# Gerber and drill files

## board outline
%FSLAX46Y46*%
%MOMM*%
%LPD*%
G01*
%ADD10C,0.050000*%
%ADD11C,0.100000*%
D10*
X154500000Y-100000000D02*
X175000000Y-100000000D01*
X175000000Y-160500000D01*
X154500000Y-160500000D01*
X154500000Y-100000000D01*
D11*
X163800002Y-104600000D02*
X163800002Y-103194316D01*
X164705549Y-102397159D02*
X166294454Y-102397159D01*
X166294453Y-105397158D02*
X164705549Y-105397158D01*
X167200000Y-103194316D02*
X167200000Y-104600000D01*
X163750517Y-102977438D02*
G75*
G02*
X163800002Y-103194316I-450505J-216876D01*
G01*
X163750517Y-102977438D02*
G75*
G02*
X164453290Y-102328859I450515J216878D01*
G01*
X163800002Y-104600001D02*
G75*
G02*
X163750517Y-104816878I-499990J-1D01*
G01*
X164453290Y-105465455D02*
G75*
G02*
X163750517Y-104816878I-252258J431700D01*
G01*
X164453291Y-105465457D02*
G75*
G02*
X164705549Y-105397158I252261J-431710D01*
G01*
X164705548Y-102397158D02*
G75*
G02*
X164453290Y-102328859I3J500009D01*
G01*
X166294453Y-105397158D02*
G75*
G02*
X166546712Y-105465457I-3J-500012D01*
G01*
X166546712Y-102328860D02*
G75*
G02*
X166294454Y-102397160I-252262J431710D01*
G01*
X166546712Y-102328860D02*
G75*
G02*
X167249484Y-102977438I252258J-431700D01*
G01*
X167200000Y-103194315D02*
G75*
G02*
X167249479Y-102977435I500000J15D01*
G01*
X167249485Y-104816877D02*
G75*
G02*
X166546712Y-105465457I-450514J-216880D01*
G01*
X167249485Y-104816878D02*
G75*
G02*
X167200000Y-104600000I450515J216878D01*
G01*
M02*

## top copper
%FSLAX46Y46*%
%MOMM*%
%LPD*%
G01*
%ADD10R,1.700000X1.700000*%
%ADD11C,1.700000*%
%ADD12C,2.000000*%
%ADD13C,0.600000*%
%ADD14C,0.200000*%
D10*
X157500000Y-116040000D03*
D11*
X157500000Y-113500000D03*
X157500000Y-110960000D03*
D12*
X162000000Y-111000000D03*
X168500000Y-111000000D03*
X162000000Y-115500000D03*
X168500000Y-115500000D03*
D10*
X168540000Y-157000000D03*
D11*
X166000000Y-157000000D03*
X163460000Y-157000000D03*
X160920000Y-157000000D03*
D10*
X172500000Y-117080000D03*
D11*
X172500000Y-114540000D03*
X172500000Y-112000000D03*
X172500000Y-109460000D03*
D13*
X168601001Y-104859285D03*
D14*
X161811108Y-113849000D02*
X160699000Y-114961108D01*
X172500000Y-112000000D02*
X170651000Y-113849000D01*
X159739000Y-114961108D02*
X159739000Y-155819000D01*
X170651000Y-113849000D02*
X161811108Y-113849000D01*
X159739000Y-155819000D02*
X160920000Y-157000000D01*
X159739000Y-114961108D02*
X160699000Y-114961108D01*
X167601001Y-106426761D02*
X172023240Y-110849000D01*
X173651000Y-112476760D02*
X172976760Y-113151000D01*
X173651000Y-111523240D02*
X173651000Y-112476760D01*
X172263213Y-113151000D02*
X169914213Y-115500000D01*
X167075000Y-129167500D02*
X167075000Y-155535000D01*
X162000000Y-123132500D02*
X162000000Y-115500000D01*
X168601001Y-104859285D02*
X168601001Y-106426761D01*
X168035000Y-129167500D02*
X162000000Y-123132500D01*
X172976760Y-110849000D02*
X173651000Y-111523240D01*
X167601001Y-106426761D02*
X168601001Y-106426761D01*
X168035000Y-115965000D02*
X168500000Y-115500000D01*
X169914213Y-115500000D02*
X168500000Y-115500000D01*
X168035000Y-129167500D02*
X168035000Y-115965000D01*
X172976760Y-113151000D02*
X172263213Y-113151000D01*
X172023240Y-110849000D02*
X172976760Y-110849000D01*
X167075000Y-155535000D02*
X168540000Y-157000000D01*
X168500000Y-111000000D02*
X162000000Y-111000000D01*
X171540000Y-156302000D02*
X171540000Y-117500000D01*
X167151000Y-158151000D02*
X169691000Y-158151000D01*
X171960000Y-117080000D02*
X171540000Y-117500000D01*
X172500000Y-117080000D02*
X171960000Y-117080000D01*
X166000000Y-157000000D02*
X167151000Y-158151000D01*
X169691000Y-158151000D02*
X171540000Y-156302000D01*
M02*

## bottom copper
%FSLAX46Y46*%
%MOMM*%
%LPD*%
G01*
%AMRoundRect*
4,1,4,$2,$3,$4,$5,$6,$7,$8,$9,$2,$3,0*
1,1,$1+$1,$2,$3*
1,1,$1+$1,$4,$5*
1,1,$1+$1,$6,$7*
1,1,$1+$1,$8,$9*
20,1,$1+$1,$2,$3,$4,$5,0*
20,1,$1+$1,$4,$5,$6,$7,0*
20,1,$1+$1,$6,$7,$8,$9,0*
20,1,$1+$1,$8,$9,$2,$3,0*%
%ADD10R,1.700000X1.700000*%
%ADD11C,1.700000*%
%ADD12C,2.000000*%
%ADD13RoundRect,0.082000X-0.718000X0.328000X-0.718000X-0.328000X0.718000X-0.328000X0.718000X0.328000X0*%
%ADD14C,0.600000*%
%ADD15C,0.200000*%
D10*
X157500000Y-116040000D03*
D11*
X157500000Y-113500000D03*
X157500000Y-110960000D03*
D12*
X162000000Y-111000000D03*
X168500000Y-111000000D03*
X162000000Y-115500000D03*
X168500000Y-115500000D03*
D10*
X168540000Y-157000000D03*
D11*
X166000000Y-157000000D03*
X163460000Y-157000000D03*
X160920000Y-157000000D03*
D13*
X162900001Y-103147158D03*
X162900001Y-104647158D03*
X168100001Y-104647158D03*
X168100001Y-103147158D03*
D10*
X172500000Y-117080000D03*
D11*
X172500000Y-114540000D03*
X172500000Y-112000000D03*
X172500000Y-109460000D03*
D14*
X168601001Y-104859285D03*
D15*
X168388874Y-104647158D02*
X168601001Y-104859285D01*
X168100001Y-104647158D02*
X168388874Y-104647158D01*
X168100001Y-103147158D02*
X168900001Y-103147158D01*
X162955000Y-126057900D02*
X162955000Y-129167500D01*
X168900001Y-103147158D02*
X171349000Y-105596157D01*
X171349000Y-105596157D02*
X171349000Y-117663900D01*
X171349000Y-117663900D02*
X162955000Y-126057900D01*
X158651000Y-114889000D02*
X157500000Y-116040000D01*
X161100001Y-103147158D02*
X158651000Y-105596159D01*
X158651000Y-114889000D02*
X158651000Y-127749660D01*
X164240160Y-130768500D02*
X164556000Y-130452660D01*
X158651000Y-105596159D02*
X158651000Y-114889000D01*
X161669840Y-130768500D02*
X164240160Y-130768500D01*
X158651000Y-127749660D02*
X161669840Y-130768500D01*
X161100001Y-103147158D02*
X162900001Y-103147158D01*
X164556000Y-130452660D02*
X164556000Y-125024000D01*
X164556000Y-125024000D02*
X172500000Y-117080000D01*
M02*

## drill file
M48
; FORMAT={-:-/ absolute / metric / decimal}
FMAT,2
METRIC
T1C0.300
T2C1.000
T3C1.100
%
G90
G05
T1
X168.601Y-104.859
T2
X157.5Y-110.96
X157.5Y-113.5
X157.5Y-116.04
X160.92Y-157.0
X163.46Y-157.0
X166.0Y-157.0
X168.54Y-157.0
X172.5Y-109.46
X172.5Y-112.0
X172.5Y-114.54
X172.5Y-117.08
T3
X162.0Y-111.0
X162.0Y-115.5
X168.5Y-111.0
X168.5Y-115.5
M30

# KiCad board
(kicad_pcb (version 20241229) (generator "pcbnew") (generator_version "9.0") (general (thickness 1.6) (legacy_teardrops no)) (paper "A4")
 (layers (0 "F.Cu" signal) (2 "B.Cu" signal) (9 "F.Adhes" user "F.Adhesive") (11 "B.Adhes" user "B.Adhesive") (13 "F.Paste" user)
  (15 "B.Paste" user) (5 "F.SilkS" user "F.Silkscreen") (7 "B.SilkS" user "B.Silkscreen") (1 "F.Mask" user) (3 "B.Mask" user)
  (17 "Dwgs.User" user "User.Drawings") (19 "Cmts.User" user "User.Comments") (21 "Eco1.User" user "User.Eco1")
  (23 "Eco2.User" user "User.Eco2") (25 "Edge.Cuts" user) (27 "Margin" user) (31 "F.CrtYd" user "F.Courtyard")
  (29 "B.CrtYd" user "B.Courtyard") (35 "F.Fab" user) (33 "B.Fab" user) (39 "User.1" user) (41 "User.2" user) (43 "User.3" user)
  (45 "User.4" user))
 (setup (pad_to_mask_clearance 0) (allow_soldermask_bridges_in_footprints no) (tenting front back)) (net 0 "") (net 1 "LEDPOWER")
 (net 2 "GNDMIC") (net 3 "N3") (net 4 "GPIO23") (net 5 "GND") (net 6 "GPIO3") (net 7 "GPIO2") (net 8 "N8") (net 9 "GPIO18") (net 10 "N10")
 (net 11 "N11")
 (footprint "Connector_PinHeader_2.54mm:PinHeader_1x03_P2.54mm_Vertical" (layer "F.Cu") (at 157.5 116.04 180)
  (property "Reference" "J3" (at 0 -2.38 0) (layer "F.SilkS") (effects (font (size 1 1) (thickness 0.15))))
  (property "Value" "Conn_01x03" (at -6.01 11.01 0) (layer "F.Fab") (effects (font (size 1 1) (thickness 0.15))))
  (pad "1" thru_hole rect (at 0 0 180) (size 1.7 1.7) (drill 1) (layers "*.Cu" "*.Mask") (remove_unused_layers no) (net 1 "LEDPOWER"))
  (pad "2" thru_hole circle (at 0 2.54 180) (size 1.7 1.7) (drill 1) (layers "*.Cu" "*.Mask") (remove_unused_layers no) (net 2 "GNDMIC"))
  (pad "3" thru_hole circle (at 0 5.08 180) (size 1.7 1.7) (drill 1) (layers "*.Cu" "*.Mask") (remove_unused_layers no) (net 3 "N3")))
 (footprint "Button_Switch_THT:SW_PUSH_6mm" (layer "F.Cu") (at 162 111)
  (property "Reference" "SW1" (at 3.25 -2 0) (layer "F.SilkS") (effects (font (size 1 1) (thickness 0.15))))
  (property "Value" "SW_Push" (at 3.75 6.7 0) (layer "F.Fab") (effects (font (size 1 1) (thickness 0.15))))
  (pad "1" thru_hole circle (at 0 0 90) (size 2 2) (drill 1.1) (layers "*.Cu" "*.Mask") (remove_unused_layers no) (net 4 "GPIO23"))
  (pad "1" thru_hole circle (at 6.5 0 90) (size 2 2) (drill 1.1) (layers "*.Cu" "*.Mask") (remove_unused_layers no) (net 4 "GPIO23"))
  (pad "2" thru_hole circle (at 0 4.5 90) (size 2 2) (drill 1.1) (layers "*.Cu" "*.Mask") (remove_unused_layers no) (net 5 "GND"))
  (pad "2" thru_hole circle (at 6.5 4.5 90) (size 2 2) (drill 1.1) (layers "*.Cu" "*.Mask") (remove_unused_layers no) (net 5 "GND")))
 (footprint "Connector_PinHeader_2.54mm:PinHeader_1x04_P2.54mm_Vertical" (layer "F.Cu") (at 168.54 157 -90)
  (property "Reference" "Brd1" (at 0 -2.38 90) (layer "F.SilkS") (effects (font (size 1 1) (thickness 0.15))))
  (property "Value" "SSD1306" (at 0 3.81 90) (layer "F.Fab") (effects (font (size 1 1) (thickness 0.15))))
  (pad "1" thru_hole rect (at 0 0 270) (size 1.7 1.7) (drill 1) (layers "*.Cu" "*.Mask") (remove_unused_layers no) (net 5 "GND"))
  (pad "2" thru_hole circle (at 0 2.54 270) (size 1.7 1.7) (drill 1) (layers "*.Cu" "*.Mask") (remove_unused_layers no) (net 1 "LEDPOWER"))
  (pad "3" thru_hole circle (at 0 5.08 270) (size 1.7 1.7) (drill 1) (layers "*.Cu" "*.Mask") (remove_unused_layers no) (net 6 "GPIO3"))
  (pad "4" thru_hole circle (at 0 7.62 270) (size 1.7 1.7) (drill 1) (layers "*.Cu" "*.Mask") (remove_unused_layers no) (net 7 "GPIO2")))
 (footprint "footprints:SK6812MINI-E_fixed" (layer "F.Cu") (at 165.5 104)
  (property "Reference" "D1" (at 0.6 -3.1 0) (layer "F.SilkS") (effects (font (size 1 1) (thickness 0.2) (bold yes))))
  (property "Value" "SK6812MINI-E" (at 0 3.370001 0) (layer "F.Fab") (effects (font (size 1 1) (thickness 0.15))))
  (fp_line (start -1.699998 0.6) (end -1.699998 -0.805684) (stroke (width 0.1) (type solid)) (layer "Edge.Cuts"))
  (fp_line (start -0.794451 -1.602841) (end 0.794454 -1.602841) (stroke (width 0.1) (type solid)) (layer "Edge.Cuts"))
  (fp_line (start 0.794453 1.397158) (end -0.794451 1.397158) (stroke (width 0.1) (type solid)) (layer "Edge.Cuts"))
  (fp_line (start 1.7 -0.805684) (end 1.7 0.6) (stroke (width 0.1) (type solid)) (layer "Edge.Cuts"))
  (fp_arc (start -1.749483 -1.022562) (mid -1.712526 -0.91691) (end -1.699998 -0.805684) (stroke (width 0.1) (type solid))
   (layer "Edge.Cuts"))
  (fp_arc (start -1.749483 -1.022562) (mid -1.63807 -1.606877) (end -1.04671 -1.671141) (stroke (width 0.1) (type solid))
   (layer "Edge.Cuts"))
  (fp_arc (start -1.699998 0.600001) (mid -1.712526 0.711226) (end -1.749483 0.816878) (stroke (width 0.1) (type solid)) (layer "Edge.Cuts"))
  (fp_arc (start -1.04671 1.465455) (mid -1.638069 1.401192) (end -1.749483 0.816878) (stroke (width 0.1) (type solid)) (layer "Edge.Cuts"))
  (fp_arc (start -1.046709 1.465457) (mid -0.925121 1.414535) (end -0.794451 1.397158) (stroke (width 0.1) (type solid)) (layer "Edge.Cuts"))
  (fp_arc (start -0.794452 -1.602842) (mid -0.925122 -1.620219) (end -1.04671 -1.671141) (stroke (width 0.1) (type solid))
   (layer "Edge.Cuts"))
  (fp_arc (start 0.794453 1.397158) (mid 0.925124 1.414535) (end 1.046712 1.465457) (stroke (width 0.1) (type solid)) (layer "Edge.Cuts"))
  (fp_arc (start 1.046712 -1.67114) (mid 0.925124 -1.620218) (end 0.794454 -1.602841) (stroke (width 0.1) (type solid)) (layer "Edge.Cuts"))
  (fp_arc (start 1.046712 -1.67114) (mid 1.638072 -1.606876) (end 1.749485 -1.022562) (stroke (width 0.1) (type solid)) (layer "Edge.Cuts"))
  (fp_arc (start 1.7 -0.805685) (mid 1.712528 -0.91691) (end 1.749485 -1.022562) (stroke (width 0.1) (type solid)) (layer "Edge.Cuts"))
  (fp_arc (start 1.749485 0.816877) (mid 1.638073 1.401193) (end 1.046712 1.465457) (stroke (width 0.1) (type solid)) (layer "Edge.Cuts"))
  (fp_arc (start 1.749485 0.816878) (mid 1.712528 0.711226) (end 1.7 0.6) (stroke (width 0.1) (type solid)) (layer "Edge.Cuts"))
  (pad "1" smd roundrect (at -2.599999 -0.852842 270) (size 0.82 1.6) (layers "B.Cu" "B.Mask" "B.Paste") (roundrect_rratio 0.1)
   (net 1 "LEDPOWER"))
  (pad "2" smd roundrect (at -2.599999 0.647158 270) (size 0.82 1.6) (layers "B.Cu" "B.Mask" "B.Paste") (roundrect_rratio 0.1) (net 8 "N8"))
  (pad "3" smd roundrect (at 2.600001 0.647158 270) (size 0.82 1.6) (layers "B.Cu" "B.Mask" "B.Paste") (roundrect_rratio 0.1) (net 5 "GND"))
  (pad "4" smd roundrect (at 2.600001 -0.852842 270) (size 0.82 1.6) (layers "B.Cu" "B.Mask" "B.Paste") (roundrect_rratio 0.1)
   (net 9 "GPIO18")))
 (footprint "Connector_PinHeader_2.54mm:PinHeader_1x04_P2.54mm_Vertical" (layer "F.Cu") (at 172.5 117.08 180)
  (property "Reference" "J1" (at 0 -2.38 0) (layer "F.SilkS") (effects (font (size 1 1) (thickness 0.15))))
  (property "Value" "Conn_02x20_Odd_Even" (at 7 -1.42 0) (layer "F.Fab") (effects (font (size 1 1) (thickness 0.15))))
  (pad "1" thru_hole rect (at 0 0 180) (size 1.7 1.7) (drill 1) (layers "*.Cu" "*.Mask") (remove_unused_layers no) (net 1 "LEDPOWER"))
  (pad "2" thru_hole circle (at 0 2.54 180) (size 1.7 1.7) (drill 1) (layers "*.Cu" "*.Mask") (remove_unused_layers no) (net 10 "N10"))
  (pad "3" thru_hole circle (at 0 5.08 180) (size 1.7 1.7) (drill 1) (layers "*.Cu" "*.Mask") (remove_unused_layers no) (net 7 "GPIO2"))
  (pad "4" thru_hole circle (at 0 7.62 180) (size 1.7 1.7) (drill 1) (layers "*.Cu" "*.Mask") (remove_unused_layers no) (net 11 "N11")))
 (gr_rect (start 154.5 100) (end 175 160.5) (stroke (width 0.05) (type default)) (fill no) (layer "Edge.Cuts"))
 (segment (start 161.811108 113.849) (end 160.699 114.961108) (width 0.2) (layer "F.Cu") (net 7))
 (segment (start 172.5 112) (end 170.651 113.849) (width 0.2) (layer "F.Cu") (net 7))
 (segment (start 159.739 114.961108) (end 159.739 155.819) (width 0.2) (layer "F.Cu") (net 7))
 (segment (start 170.651 113.849) (end 161.811108 113.849) (width 0.2) (layer "F.Cu") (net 7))
 (segment (start 159.739 155.819) (end 160.92 157) (width 0.2) (layer "F.Cu") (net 7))
 (segment (start 159.739 114.961108) (end 160.699 114.961108) (width 0.2) (layer "F.Cu") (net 7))
 (segment (start 167.601001 106.426761) (end 172.02324 110.849) (width 0.2) (layer "F.Cu") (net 5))
 (segment (start 173.651 112.47676) (end 172.97676 113.151) (width 0.2) (layer "F.Cu") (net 5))
 (segment (start 173.651 111.52324) (end 173.651 112.47676) (width 0.2) (layer "F.Cu") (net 5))
 (segment (start 172.263213 113.151) (end 169.914213 115.5) (width 0.2) (layer "F.Cu") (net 5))
 (segment (start 167.075 129.1675) (end 167.075 155.535) (width 0.2) (layer "F.Cu") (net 5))
 (segment (start 162 123.1325) (end 162 115.5) (width 0.2) (layer "F.Cu") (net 5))
 (segment (start 168.601001 104.859285) (end 168.601001 106.426761) (width 0.2) (layer "F.Cu") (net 5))
 (segment (start 168.035 129.1675) (end 162 123.1325) (width 0.2) (layer "F.Cu") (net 5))
 (segment (start 172.97676 110.849) (end 173.651 111.52324) (width 0.2) (layer "F.Cu") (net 5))
 (segment (start 167.601001 106.426761) (end 168.601001 106.426761) (width 0.2) (layer "F.Cu") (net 5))
 (segment (start 168.035 115.965) (end 168.5 115.5) (width 0.2) (layer "F.Cu") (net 5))
 (segment (start 169.914213 115.5) (end 168.5 115.5) (width 0.2) (layer "F.Cu") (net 5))
 (segment (start 168.035 129.1675) (end 168.035 115.965) (width 0.2) (layer "F.Cu") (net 5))
 (segment (start 172.97676 113.151) (end 172.263213 113.151) (width 0.2) (layer "F.Cu") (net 5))
 (segment (start 172.02324 110.849) (end 172.97676 110.849) (width 0.2) (layer "F.Cu") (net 5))
 (segment (start 167.075 155.535) (end 168.54 157) (width 0.2) (layer "F.Cu") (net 5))
 (via (at 168.601001 104.859285) (size 0.6) (drill 0.3) (layers "F.Cu" "B.Cu") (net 5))
 (segment (start 168.388874 104.647158) (end 168.601001 104.859285) (width 0.2) (layer "B.Cu") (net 5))
 (segment (start 168.100001 104.647158) (end 168.388874 104.647158) (width 0.2) (layer "B.Cu") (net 5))
 (segment (start 168.100001 103.147158) (end 168.900001 103.147158) (width 0.2) (layer "B.Cu") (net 9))
 (segment (start 162.955 126.0579) (end 162.955 129.1675) (width 0.2) (layer "B.Cu") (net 9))
 (segment (start 168.900001 103.147158) (end 171.349 105.596157) (width 0.2) (layer "B.Cu") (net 9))
 (segment (start 171.349 105.596157) (end 171.349 117.6639) (width 0.2) (layer "B.Cu") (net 9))
 (segment (start 171.349 117.6639) (end 162.955 126.0579) (width 0.2) (layer "B.Cu") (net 9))
 (segment (start 168.5 111) (end 162 111) (width 0.2) (layer "F.Cu") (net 4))
 (segment (start 171.54 156.302) (end 171.54 117.5) (width 0.2) (layer "F.Cu") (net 1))
 (segment (start 167.151 158.151) (end 169.691 158.151) (width 0.2) (layer "F.Cu") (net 1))
 (segment (start 171.96 117.08) (end 171.54 117.5) (width 0.2) (layer "F.Cu") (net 1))
 (segment (start 172.5 117.08) (end 171.96 117.08) (width 0.2) (layer "F.Cu") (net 1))
 (segment (start 166 157) (end 167.151 158.151) (width 0.2) (layer "F.Cu") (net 1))
 (segment (start 169.691 158.151) (end 171.54 156.302) (width 0.2) (layer "F.Cu") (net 1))
 (segment (start 158.651 114.889) (end 157.5 116.04) (width 0.2) (layer "B.Cu") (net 1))
 (segment (start 161.100001 103.147158) (end 158.651 105.596159) (width 0.2) (layer "B.Cu") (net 1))
 (segment (start 158.651 114.889) (end 158.651 127.74966) (width 0.2) (layer "B.Cu") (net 1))
 (segment (start 164.24016 130.7685) (end 164.556 130.45266) (width 0.2) (layer "B.Cu") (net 1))
 (segment (start 158.651 105.596159) (end 158.651 114.889) (width 0.2) (layer "B.Cu") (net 1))
 (segment (start 161.66984 130.7685) (end 164.24016 130.7685) (width 0.2) (layer "B.Cu") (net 1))
 (segment (start 158.651 127.74966) (end 161.66984 130.7685) (width 0.2) (layer "B.Cu") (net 1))
 (segment (start 161.100001 103.147158) (end 162.900001 103.147158) (width 0.2) (layer "B.Cu") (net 1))
 (segment (start 164.556 130.45266) (end 164.556 125.024) (width 0.2) (layer "B.Cu") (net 1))
 (segment (start 164.556 125.024) (end 172.5 117.08) (width 0.2) (layer "B.Cu") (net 1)))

